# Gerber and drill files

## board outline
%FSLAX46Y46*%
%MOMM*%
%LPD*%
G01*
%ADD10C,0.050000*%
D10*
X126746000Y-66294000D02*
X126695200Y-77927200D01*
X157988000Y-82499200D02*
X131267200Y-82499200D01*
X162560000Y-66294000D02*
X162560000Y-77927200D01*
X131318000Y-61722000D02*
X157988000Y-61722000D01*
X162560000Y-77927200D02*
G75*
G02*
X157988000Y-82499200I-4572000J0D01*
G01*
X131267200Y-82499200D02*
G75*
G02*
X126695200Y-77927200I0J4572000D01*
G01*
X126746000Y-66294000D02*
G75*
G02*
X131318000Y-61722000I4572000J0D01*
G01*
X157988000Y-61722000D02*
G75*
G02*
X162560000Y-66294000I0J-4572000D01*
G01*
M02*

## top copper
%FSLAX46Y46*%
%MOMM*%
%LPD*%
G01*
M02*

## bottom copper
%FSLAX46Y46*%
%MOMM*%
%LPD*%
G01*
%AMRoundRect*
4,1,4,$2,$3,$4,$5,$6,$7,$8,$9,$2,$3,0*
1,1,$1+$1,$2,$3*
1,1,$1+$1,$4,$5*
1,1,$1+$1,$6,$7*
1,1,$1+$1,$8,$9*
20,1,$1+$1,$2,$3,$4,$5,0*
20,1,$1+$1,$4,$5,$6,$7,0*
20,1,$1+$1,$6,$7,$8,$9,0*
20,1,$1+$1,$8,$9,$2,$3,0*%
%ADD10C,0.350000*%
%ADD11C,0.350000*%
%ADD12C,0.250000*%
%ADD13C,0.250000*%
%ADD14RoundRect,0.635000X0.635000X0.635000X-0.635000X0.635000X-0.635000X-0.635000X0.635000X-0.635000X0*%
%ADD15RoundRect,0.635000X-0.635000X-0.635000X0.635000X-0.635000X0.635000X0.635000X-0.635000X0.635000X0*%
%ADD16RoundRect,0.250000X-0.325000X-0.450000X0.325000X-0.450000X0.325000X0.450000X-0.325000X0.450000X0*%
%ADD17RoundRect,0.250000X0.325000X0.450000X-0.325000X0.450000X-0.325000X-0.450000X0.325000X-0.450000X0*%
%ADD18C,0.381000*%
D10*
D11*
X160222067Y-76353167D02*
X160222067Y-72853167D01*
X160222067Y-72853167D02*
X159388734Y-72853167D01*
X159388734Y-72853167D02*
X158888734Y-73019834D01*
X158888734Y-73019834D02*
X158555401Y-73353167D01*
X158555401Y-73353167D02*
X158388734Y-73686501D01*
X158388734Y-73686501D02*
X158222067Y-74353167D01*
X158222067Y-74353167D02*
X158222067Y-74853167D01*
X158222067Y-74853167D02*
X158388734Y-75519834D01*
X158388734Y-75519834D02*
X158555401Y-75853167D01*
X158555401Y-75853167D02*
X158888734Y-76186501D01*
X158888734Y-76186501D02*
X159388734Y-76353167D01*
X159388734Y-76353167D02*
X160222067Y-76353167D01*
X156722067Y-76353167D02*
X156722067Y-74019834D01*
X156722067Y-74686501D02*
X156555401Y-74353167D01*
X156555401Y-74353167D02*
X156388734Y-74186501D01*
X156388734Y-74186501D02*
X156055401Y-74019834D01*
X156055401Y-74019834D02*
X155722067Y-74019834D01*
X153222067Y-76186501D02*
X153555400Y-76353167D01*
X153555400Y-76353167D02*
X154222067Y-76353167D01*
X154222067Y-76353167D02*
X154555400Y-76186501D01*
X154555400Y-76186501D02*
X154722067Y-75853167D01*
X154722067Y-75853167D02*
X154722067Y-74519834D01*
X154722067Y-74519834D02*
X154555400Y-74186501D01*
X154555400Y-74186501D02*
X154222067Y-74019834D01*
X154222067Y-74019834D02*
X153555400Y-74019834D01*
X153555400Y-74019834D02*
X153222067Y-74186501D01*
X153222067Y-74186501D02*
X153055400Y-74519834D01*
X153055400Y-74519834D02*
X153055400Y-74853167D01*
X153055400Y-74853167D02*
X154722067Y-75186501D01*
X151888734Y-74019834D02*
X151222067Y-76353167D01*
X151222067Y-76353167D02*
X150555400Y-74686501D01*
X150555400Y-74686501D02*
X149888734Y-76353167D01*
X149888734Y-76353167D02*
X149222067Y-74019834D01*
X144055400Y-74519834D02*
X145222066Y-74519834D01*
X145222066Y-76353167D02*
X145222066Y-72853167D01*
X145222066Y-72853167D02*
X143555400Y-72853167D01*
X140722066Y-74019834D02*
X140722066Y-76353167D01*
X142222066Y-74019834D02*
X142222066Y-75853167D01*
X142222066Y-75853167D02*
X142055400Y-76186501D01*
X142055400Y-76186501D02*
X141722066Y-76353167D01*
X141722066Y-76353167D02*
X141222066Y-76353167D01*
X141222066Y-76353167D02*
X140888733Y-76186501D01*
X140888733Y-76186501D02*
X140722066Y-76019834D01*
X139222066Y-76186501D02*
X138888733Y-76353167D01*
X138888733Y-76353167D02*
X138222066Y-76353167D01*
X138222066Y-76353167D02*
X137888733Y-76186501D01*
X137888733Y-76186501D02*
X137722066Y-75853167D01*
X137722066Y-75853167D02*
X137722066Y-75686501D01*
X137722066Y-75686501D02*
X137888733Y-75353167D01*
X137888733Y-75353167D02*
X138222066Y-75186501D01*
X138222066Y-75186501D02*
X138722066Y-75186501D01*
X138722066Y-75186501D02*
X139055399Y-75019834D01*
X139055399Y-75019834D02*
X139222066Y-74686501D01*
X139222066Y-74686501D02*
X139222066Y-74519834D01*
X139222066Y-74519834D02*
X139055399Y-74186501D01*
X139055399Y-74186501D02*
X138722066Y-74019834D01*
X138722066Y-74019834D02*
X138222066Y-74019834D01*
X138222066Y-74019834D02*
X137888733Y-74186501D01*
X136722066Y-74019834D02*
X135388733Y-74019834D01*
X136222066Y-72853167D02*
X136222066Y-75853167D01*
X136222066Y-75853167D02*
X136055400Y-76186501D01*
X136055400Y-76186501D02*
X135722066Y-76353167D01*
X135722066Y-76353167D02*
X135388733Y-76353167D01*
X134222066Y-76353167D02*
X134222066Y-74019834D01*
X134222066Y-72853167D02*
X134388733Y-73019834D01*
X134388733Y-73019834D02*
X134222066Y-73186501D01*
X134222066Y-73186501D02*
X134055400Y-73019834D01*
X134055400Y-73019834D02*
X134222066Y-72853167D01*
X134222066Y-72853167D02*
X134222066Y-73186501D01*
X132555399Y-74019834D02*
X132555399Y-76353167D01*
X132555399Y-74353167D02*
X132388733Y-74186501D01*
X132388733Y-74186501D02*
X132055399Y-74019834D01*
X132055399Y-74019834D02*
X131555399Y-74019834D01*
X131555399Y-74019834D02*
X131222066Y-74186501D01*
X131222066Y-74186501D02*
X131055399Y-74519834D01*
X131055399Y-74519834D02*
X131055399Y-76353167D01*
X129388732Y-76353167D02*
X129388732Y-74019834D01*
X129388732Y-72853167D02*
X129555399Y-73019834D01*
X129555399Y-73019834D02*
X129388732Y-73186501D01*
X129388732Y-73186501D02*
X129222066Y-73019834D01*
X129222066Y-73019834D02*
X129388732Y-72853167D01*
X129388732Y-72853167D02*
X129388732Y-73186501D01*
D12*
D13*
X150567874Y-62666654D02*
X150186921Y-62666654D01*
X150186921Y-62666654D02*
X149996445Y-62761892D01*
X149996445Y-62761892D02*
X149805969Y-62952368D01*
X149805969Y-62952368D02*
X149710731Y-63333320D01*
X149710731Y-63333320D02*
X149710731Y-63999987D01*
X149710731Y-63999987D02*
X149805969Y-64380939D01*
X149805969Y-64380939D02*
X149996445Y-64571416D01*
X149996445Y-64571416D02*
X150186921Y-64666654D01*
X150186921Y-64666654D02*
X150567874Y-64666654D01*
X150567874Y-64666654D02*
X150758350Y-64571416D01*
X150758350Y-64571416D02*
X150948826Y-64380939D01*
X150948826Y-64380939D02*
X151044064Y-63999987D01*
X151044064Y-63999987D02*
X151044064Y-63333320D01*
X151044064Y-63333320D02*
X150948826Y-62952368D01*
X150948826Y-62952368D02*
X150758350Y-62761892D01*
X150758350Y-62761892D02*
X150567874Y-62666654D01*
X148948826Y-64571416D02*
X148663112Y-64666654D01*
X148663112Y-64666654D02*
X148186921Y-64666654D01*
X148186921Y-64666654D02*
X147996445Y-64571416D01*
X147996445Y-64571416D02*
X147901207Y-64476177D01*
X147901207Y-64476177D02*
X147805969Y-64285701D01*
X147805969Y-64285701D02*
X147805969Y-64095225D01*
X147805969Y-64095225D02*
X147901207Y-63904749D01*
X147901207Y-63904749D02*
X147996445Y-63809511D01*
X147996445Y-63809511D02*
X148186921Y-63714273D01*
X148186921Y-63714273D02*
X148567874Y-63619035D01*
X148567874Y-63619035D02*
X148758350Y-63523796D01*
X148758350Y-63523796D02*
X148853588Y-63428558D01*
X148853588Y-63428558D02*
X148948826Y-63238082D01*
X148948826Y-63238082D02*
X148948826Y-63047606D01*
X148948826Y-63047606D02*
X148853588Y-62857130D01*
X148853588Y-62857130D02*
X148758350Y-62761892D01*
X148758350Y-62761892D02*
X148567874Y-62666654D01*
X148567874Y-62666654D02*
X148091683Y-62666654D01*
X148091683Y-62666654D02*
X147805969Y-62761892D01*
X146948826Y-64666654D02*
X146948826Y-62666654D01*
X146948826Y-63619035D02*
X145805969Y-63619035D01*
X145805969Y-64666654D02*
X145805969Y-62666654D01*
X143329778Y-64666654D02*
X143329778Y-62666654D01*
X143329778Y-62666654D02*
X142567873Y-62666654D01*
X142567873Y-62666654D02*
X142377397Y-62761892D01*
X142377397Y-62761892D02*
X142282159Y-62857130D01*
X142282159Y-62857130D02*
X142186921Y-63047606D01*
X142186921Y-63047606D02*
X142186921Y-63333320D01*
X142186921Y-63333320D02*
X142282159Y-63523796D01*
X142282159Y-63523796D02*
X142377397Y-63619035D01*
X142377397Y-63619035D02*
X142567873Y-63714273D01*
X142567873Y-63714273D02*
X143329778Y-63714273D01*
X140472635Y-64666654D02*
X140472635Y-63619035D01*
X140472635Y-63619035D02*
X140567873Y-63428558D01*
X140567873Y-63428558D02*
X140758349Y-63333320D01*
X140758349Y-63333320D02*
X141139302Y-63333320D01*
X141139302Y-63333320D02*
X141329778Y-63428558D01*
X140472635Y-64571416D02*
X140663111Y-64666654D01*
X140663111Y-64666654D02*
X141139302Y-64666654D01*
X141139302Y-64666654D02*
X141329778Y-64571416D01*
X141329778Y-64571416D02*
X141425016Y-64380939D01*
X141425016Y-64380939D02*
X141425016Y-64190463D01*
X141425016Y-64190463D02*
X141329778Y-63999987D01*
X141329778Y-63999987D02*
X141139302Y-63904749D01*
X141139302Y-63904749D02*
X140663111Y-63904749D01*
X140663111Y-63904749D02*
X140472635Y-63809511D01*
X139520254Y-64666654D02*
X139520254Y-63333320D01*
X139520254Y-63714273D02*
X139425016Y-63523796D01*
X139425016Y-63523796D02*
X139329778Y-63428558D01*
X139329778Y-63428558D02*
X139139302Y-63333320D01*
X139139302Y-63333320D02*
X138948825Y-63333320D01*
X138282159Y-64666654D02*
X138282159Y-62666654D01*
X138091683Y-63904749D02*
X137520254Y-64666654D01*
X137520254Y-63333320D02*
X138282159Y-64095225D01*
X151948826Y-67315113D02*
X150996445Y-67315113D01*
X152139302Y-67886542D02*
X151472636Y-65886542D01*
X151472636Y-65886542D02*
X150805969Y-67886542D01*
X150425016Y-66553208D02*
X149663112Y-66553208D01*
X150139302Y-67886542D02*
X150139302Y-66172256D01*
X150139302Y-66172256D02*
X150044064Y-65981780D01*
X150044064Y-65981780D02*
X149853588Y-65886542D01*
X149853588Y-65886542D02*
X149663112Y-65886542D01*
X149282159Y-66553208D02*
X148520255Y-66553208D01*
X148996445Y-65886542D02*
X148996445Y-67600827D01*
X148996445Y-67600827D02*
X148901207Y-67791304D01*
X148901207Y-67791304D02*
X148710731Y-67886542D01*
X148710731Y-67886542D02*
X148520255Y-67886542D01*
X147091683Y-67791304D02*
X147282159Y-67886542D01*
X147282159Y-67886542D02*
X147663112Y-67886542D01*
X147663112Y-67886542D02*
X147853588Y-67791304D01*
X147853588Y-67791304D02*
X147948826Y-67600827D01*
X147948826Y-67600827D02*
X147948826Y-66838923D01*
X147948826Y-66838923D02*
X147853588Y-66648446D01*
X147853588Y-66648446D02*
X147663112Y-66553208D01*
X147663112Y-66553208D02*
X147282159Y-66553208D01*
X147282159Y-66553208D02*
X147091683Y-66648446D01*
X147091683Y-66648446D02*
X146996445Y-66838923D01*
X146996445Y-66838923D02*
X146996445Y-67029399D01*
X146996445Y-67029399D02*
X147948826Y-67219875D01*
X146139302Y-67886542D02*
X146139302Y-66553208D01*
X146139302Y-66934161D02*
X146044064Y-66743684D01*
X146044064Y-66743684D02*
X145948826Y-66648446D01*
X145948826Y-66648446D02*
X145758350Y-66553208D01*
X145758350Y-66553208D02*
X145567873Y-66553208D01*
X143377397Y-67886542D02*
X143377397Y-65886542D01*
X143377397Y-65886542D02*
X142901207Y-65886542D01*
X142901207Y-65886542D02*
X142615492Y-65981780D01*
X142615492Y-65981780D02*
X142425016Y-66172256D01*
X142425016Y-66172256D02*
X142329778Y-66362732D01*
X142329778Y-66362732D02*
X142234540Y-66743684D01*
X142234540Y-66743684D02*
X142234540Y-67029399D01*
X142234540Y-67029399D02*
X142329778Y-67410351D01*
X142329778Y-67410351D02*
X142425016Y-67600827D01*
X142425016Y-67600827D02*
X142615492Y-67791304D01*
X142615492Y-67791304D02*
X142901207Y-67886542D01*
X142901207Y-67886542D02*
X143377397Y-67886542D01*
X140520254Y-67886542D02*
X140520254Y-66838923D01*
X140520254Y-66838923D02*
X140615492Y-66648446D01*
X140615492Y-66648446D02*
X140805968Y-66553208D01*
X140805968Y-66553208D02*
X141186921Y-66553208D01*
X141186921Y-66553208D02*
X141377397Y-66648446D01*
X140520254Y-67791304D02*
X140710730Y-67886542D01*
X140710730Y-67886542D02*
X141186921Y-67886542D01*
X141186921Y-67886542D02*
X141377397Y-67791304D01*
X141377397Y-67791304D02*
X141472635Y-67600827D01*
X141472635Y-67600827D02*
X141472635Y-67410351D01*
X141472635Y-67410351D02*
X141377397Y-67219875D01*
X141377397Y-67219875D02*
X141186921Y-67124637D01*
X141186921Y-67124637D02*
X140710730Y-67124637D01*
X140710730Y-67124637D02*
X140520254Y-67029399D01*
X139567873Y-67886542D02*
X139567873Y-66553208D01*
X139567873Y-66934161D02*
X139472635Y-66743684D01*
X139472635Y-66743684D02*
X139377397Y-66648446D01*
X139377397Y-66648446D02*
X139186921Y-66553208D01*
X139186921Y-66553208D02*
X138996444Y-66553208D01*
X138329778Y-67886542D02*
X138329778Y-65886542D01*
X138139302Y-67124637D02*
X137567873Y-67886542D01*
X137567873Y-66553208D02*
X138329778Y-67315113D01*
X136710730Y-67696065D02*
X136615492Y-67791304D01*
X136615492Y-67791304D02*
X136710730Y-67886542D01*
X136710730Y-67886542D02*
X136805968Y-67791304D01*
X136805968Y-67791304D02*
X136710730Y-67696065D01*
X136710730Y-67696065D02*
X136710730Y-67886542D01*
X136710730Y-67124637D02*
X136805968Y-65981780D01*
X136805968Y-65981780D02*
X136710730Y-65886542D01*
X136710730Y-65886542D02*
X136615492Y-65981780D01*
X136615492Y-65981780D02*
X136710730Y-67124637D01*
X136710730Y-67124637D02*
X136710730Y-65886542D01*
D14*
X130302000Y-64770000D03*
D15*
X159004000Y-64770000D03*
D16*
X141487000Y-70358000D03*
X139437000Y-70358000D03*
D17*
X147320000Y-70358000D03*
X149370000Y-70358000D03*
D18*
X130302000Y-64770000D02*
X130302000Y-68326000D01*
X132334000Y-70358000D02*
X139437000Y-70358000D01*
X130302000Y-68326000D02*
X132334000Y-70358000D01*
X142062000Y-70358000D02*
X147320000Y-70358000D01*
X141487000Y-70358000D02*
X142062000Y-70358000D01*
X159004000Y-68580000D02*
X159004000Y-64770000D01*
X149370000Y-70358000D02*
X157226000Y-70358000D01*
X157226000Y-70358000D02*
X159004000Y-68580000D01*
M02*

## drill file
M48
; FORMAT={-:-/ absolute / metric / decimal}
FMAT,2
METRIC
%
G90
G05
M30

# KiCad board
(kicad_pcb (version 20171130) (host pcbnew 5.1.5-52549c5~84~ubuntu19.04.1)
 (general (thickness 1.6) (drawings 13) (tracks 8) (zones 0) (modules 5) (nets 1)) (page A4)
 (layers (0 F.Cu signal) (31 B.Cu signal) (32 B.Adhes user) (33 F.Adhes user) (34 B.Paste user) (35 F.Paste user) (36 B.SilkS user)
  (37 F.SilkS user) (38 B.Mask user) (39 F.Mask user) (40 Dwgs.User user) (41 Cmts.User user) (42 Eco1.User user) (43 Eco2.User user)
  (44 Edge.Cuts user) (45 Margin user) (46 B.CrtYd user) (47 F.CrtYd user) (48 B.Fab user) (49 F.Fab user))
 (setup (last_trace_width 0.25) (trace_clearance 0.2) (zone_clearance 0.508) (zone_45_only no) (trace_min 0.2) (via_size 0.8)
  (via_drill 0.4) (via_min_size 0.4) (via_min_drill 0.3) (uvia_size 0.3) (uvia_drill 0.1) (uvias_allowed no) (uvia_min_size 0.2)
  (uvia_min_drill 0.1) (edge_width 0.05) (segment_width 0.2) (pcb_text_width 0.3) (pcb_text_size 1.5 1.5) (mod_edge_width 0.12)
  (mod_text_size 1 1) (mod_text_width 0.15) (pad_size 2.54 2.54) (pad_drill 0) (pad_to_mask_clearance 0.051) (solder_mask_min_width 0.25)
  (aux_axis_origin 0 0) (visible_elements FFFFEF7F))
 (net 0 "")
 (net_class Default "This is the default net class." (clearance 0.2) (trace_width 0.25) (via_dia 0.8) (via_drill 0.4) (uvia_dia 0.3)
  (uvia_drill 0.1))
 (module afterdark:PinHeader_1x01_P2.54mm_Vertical (layer F.Cu) (at 130.302 64.77 180)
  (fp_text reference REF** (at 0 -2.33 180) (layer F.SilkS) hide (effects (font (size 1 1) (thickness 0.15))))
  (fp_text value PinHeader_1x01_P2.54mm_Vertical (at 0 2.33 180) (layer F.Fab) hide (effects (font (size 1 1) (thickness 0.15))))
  (pad 1 smd roundrect (at 0 0 180) (size 2.54 2.54) (layers B.Cu B.Paste B.Mask) (roundrect_rratio 0.25)))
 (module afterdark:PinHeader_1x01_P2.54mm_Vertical (layer B.Cu) (at 159.004 64.77)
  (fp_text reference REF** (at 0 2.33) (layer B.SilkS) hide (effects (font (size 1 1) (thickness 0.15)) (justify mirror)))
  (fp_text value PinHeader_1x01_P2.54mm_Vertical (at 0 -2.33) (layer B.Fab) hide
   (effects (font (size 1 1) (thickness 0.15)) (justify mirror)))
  (pad 1 smd roundrect (at 0 0) (size 2.54 2.54) (layers B.Cu B.Paste B.Mask) (roundrect_rratio 0.25)))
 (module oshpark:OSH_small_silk (layer F.Cu) (at 144.4244 71.8312)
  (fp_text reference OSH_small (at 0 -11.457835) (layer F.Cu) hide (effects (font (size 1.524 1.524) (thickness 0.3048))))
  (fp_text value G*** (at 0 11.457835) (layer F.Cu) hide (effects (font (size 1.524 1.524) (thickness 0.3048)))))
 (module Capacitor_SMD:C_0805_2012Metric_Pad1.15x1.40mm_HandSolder (layer B.Cu) (at 140.462 70.358)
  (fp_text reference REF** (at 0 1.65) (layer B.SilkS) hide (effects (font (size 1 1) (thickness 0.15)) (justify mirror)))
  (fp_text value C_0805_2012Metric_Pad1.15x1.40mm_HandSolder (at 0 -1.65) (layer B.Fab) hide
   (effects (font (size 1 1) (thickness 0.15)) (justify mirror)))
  (pad 2 smd roundrect (at 1.025 0) (size 1.15 1.4) (layers B.Cu B.Paste B.Mask) (roundrect_rratio 0.217391))
  (pad 1 smd roundrect (at -1.025 0) (size 1.15 1.4) (layers B.Cu B.Paste B.Mask) (roundrect_rratio 0.217391)))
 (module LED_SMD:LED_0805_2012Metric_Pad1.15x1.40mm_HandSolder (layer B.Cu) (at 148.345 70.358 180)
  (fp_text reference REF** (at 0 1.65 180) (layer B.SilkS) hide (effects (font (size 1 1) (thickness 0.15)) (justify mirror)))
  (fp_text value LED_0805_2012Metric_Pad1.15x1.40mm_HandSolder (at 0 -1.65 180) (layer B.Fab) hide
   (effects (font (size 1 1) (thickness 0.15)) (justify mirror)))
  (pad 2 smd roundrect (at 1.025 0 180) (size 1.15 1.4) (layers B.Cu B.Paste B.Mask) (roundrect_rratio 0.217391))
  (pad 1 smd roundrect (at -1.025 0 180) (size 1.15 1.4) (layers B.Cu B.Paste B.Mask) (roundrect_rratio 0.217391)))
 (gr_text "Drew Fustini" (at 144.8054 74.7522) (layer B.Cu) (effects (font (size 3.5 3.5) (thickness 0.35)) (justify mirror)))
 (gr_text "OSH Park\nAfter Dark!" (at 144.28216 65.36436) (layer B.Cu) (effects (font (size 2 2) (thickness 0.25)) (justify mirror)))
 (gr_line (start 126.746 66.294) (end 126.6952 77.9272) (layer Edge.Cuts) (width 0.05))
 (gr_line (start 157.988 82.4992) (end 131.2672 82.4992) (layer Edge.Cuts) (width 0.05))
 (gr_line (start 162.56 66.294) (end 162.56 77.9272) (layer Edge.Cuts) (width 0.05))
 (gr_line (start 131.318 61.722) (end 157.988 61.722) (layer Edge.Cuts) (width 0.05))
 (gr_arc (start 157.988 77.9272) (end 157.988 82.4992) (angle -90) (layer Edge.Cuts) (width 0.05))
 (gr_arc (start 131.2672 77.9272) (end 126.6952 77.9272) (angle -90) (layer Edge.Cuts) (width 0.05))
 (gr_arc (start 131.318 66.294) (end 131.318 61.722) (angle -90) (layer Edge.Cuts) (width 0.05))
 (gr_arc (start 157.988 66.294) (end 162.56 66.294) (angle -90) (layer Edge.Cuts) (width 0.05))
 (segment (start 130.302 64.77) (end 130.302 68.326) (width 0.381) (layer B.Cu) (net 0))
 (segment (start 132.334 70.358) (end 139.437 70.358) (width 0.381) (layer B.Cu) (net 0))
 (segment (start 130.302 68.326) (end 132.334 70.358) (width 0.381) (layer B.Cu) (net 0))
 (segment (start 142.062 70.358) (end 147.32 70.358) (width 0.381) (layer B.Cu) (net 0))
 (segment (start 141.487 70.358) (end 142.062 70.358) (width 0.381) (layer B.Cu) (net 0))
 (segment (start 159.004 68.58) (end 159.004 64.77) (width 0.381) (layer B.Cu) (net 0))
 (segment (start 149.37 70.358) (end 157.226 70.358) (width 0.381) (layer B.Cu) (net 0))
 (segment (start 157.226 70.358) (end 159.004 68.58) (width 0.381) (layer B.Cu) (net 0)))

